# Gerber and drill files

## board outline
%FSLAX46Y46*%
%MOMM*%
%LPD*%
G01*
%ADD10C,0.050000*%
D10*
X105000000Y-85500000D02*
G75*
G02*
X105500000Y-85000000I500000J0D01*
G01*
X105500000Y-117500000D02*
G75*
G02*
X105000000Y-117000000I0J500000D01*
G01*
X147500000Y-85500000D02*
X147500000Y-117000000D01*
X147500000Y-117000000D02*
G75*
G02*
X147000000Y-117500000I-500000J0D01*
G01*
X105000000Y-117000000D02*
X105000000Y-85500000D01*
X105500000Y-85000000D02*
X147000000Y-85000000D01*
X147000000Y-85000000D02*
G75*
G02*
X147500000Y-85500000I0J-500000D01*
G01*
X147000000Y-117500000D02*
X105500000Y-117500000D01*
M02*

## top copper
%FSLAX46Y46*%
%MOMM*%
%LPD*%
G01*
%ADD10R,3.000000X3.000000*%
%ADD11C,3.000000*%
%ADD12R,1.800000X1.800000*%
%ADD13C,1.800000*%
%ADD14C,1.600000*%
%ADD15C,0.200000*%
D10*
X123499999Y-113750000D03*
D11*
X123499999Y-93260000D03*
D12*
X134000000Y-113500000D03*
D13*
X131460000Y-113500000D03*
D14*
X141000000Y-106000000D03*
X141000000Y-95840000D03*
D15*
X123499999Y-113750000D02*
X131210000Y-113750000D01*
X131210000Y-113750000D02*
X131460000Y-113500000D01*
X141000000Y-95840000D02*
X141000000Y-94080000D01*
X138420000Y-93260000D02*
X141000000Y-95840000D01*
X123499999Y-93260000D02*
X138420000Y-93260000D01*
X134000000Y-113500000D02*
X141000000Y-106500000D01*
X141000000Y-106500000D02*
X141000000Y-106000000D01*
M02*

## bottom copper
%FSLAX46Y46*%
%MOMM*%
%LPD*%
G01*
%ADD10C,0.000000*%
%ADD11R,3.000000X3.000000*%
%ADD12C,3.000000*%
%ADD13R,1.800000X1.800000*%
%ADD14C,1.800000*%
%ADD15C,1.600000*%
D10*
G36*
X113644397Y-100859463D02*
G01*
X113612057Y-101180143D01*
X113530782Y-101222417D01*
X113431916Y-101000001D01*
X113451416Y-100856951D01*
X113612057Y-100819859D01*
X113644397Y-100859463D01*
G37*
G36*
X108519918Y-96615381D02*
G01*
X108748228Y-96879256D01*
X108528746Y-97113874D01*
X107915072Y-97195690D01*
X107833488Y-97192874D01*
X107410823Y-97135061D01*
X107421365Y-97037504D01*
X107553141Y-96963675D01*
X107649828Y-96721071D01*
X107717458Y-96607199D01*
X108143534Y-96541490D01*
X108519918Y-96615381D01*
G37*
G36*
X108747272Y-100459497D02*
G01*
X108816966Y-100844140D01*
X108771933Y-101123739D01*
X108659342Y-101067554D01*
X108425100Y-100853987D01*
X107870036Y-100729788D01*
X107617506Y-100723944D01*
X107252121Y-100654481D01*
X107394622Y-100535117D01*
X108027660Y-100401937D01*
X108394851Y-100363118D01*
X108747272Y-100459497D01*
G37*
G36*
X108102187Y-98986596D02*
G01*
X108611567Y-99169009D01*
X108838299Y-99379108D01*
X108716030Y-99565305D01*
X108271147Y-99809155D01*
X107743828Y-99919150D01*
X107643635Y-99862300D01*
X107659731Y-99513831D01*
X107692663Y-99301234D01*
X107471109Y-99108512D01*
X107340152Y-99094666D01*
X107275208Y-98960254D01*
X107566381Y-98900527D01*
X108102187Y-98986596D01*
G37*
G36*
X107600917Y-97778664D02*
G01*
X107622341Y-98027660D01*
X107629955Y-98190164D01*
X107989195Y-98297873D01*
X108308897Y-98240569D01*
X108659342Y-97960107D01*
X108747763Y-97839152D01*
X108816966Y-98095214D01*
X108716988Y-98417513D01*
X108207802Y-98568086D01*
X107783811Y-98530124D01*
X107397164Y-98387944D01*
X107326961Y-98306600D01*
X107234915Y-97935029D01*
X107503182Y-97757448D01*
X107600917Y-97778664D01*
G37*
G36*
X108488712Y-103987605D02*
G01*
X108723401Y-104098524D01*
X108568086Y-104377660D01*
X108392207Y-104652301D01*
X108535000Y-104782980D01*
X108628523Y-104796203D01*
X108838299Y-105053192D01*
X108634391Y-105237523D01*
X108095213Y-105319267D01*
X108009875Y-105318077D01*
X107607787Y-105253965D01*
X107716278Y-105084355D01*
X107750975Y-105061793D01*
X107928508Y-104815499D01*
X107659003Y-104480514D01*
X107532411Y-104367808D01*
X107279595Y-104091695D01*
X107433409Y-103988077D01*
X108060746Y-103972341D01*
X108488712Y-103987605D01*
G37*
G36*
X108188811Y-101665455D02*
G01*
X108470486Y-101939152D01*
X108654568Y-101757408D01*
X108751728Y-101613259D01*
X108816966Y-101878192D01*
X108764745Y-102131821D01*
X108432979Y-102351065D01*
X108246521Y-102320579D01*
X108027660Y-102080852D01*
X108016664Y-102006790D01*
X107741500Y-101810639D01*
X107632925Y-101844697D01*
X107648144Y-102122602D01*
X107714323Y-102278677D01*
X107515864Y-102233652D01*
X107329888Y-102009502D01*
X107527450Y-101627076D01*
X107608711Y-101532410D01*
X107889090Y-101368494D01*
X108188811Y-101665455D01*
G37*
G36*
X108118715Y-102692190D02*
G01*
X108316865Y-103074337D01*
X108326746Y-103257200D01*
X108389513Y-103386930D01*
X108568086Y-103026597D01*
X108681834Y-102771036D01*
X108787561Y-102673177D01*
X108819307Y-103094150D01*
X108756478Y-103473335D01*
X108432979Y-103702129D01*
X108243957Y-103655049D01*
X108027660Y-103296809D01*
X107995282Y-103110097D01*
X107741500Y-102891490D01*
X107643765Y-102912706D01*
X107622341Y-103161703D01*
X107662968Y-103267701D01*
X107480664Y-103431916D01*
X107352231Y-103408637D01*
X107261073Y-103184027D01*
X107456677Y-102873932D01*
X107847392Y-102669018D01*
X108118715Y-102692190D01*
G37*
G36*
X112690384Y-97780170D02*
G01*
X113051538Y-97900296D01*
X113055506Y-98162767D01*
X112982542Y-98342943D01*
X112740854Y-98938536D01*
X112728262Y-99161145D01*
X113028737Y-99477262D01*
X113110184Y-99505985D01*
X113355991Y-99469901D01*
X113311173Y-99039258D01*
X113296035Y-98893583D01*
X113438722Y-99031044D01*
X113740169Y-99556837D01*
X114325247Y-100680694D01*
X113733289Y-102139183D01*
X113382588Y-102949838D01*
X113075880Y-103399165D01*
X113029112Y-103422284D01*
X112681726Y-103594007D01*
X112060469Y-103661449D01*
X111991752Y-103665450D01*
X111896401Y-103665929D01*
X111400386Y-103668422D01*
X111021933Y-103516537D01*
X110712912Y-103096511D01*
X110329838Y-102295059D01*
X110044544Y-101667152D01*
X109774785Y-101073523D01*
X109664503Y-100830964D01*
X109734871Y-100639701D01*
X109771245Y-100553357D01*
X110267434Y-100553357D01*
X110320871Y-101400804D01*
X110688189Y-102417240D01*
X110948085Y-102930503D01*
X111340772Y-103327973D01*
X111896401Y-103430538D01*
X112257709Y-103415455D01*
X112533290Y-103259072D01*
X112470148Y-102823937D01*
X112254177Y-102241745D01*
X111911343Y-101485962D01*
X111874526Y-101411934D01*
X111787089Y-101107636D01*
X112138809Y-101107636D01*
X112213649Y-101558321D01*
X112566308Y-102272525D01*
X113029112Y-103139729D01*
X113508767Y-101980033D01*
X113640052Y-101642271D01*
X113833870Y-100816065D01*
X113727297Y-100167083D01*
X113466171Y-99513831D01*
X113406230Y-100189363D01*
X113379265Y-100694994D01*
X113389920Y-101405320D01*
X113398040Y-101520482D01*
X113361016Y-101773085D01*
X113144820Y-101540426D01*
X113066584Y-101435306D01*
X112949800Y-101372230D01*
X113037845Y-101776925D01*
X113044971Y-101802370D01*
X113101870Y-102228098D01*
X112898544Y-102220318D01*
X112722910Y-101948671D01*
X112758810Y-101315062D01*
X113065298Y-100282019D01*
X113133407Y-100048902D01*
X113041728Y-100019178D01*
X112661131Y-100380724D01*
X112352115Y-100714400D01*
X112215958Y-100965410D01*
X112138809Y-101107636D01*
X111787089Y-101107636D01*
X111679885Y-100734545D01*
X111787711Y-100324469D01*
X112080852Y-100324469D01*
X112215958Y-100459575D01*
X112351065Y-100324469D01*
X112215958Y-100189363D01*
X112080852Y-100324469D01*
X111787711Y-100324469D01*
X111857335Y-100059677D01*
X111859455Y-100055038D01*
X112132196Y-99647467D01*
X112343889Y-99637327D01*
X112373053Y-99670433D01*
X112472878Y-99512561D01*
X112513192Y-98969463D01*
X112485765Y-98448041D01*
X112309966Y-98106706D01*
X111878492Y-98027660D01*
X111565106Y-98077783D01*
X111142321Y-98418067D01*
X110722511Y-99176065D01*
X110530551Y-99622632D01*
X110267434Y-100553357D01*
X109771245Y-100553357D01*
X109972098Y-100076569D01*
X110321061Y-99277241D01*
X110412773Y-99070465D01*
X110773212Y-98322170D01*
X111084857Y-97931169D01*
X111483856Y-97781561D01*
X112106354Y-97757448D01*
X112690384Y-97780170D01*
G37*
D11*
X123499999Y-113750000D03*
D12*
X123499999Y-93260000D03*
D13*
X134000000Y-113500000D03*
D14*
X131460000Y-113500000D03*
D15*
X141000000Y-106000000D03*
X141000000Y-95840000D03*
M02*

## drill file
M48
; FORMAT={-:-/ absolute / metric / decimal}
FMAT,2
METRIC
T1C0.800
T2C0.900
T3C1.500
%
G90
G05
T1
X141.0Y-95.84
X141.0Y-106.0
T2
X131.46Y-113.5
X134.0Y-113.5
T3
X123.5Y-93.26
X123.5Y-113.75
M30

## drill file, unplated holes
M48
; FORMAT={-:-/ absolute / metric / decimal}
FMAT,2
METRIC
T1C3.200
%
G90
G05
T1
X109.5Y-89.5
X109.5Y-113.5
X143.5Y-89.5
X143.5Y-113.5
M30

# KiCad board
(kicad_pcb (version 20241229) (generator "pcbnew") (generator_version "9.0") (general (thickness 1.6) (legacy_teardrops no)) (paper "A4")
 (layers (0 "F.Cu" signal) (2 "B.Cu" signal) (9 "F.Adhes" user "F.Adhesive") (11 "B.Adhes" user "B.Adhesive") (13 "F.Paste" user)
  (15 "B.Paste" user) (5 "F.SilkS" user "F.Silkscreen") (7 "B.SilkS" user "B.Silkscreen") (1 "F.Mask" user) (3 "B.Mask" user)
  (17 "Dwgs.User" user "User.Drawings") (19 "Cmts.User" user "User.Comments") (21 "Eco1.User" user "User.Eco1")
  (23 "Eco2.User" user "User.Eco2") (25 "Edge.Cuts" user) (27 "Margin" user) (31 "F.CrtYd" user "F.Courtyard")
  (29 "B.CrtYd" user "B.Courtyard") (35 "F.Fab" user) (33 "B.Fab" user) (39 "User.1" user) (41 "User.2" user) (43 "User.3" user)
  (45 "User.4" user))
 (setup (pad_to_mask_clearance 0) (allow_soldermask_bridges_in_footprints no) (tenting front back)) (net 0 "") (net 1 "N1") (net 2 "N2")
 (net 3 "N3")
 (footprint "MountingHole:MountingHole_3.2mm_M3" (layer "F.Cu") (at 143.5 89.5)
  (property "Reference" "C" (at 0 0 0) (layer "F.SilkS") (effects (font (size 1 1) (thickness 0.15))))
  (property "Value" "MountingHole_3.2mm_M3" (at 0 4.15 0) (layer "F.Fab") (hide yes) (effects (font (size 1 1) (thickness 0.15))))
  (pad "" np_thru_hole circle (at 0 0) (size 3.2 3.2) (drill 3.2) (layers "*.Cu" "*.Mask")))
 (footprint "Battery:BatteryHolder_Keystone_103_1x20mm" (layer "F.Cu") (at 123.499999 113.75 90)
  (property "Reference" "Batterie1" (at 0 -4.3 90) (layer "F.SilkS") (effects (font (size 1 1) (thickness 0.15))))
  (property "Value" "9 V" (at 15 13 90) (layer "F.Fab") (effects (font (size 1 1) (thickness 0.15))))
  (pad "1" thru_hole rect (at 0 0 90) (size 3 3) (drill 1.5) (layers "*.Cu" "*.Mask") (remove_unused_layers no) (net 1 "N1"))
  (pad "2" thru_hole circle (at 20.49 0 90) (size 3 3) (drill 1.5) (layers "*.Cu" "*.Mask") (remove_unused_layers no) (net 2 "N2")))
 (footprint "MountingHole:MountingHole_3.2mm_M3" (layer "F.Cu") (at 143.5 113.5)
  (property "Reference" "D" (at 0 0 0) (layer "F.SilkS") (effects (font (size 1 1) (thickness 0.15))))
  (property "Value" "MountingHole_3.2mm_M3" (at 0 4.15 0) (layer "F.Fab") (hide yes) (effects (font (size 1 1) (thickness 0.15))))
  (pad "" np_thru_hole circle (at 0 0) (size 3.2 3.2) (drill 3.2) (layers "*.Cu" "*.Mask")))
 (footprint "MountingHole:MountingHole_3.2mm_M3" (layer "F.Cu") (at 109.5 113.5)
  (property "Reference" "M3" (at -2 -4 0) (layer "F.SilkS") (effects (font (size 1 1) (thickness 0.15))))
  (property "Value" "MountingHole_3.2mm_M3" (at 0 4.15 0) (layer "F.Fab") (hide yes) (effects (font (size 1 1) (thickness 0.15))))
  (pad "" np_thru_hole circle (at 0 0) (size 3.2 3.2) (drill 3.2) (layers "*.Cu" "*.Mask")))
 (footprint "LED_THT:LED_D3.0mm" (layer "F.Cu") (at 134 113.5 180)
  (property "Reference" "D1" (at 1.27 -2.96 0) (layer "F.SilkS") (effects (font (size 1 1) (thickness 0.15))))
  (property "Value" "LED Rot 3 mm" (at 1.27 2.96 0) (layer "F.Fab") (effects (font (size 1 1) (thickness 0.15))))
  (pad "1" thru_hole rect (at 0 0 180) (size 1.8 1.8) (drill 0.9) (layers "*.Cu" "*.Mask") (remove_unused_layers no) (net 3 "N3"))
  (pad "2" thru_hole circle (at 2.54 0 180) (size 1.8 1.8) (drill 0.9) (layers "*.Cu" "*.Mask") (remove_unused_layers no) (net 1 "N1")))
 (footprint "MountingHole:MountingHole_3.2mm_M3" (layer "F.Cu") (at 109.5 89.5)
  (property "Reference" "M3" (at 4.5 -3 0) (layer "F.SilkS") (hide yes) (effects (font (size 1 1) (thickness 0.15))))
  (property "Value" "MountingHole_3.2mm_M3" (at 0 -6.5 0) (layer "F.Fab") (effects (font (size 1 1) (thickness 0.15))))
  (pad "" np_thru_hole circle (at 0 0) (size 3.2 3.2) (drill 3.2) (layers "*.Cu" "*.Mask")))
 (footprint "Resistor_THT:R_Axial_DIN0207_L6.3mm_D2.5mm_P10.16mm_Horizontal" (layer "F.Cu") (at 141 106 90)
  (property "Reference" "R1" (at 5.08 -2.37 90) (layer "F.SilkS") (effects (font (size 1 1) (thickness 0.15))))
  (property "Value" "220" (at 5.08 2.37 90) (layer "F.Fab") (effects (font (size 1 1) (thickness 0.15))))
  (pad "1" thru_hole circle (at 0 0 90) (size 1.6 1.6) (drill 0.8) (layers "*.Cu" "*.Mask") (remove_unused_layers no) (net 3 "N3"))
  (pad "2" thru_hole circle (at 10.16 0 90) (size 1.6 1.6) (drill 0.8) (layers "*.Cu" "*.Mask") (remove_unused_layers no) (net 2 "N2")))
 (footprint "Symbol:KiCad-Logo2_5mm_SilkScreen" (layer "B.Cu") (at 124 99 180)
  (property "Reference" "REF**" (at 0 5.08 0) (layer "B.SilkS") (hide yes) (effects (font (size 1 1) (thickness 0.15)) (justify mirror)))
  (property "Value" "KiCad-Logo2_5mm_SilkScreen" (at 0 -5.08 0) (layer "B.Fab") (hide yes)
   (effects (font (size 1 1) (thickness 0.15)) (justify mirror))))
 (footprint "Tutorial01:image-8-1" (layer "B.Cu") (at 111 101 90)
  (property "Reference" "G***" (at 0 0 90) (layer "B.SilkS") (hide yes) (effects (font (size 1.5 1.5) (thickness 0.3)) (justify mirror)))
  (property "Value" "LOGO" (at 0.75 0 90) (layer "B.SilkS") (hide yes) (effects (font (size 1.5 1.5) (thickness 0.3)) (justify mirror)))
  (fp_poly
   (pts (xy 0.180141 2.612057) (xy 0.143049 2.451416) (xy -0.000001 2.431916) (xy -0.222417 2.530782) (xy -0.180143 2.612057)
    (xy 0.140537 2.644397))
   (stroke (width 0) (type solid)) (fill yes) (layer "B.Cu"))
  (fp_poly
   (pts (xy 4.384619 -2.480082) (xy 4.45851 -2.856466) (xy 4.392801 -3.282542) (xy 4.278929 -3.350172) (xy 4.036325 -3.446859)
    (xy 3.962496 -3.578635) (xy 3.864939 -3.589177) (xy 3.807126 -3.166512) (xy 3.80431 -3.084928) (xy 3.886126 -2.471254)
    (xy 4.120744 -2.251772))
   (stroke (width 0) (type solid)) (fill yes) (layer "B.Cu"))
  (fp_poly
   (pts (xy 0.540503 -2.252728) (xy 0.636882 -2.605149) (xy 0.598063 -2.97234) (xy 0.464883 -3.605378) (xy 0.345519 -3.747879)
    (xy 0.276056 -3.382494) (xy 0.270212 -3.129964) (xy 0.146013 -2.5749) (xy -0.067554 -2.340658) (xy -0.123739 -2.228067)
    (xy 0.15586 -2.183034))
   (stroke (width 0) (type solid)) (fill yes) (layer "B.Cu"))
  (fp_poly
   (pts (xy 1.830991 -2.388433) (xy 2.013404 -2.897813) (xy 2.099473 -3.433619) (xy 2.039746 -3.724792) (xy 1.905334 -3.659848)
    (xy 1.891488 -3.528891) (xy 1.698766 -3.307337) (xy 1.486169 -3.340269) (xy 1.1377 -3.356365) (xy 1.08085 -3.256172)
    (xy 1.190845 -2.728853) (xy 1.434695 -2.28397) (xy 1.620892 -2.161701))
   (stroke (width 0) (type solid)) (fill yes) (layer "B.Cu"))
  (fp_poly
   (pts (xy 3.160848 -2.252237) (xy 3.039893 -2.340658) (xy 2.759431 -2.691103) (xy 2.702127 -3.010805) (xy 2.809836 -3.370045)
    (xy 2.97234 -3.377659) (xy 3.221336 -3.399083) (xy 3.242552 -3.496818) (xy 3.064971 -3.765085) (xy 2.6934 -3.673039)
    (xy 2.612056 -3.602836) (xy 2.469876 -3.216189) (xy 2.431914 -2.792198) (xy 2.582487 -2.283012) (xy 2.904786 -2.183034))
   (stroke (width 0) (type solid)) (fill yes) (layer "B.Cu"))
  (fp_poly
   (pts (xy -3.796203 -2.371477) (xy -3.78298 -2.465) (xy -3.652301 -2.607793) (xy -3.37766 -2.431914) (xy -3.098524 -2.276599)
    (xy -2.987605 -2.511288) (xy -2.972341 -2.939254) (xy -2.988077 -3.566591) (xy -3.091695 -3.720405) (xy -3.367808 -3.467589)
    (xy -3.480514 -3.340997) (xy -3.815499 -3.071492) (xy -4.061793 -3.249025) (xy -4.084355 -3.283722) (xy -4.253965 -3.392213)
    (xy -4.318077 -2.990125) (xy -4.319267 -2.904787) (xy -4.237523 -2.365609) (xy -4.053192 -2.161701))
   (stroke (width 0) (type solid)) (fill yes) (layer "B.Cu"))
  (fp_poly
   (pts (xy -0.613259 -2.248272) (xy -0.757408 -2.345432) (xy -0.939152 -2.529514) (xy -0.665455 -2.811189) (xy -0.368494 -3.11091)
    (xy -0.53241 -3.391289) (xy -0.627076 -3.47255) (xy -1.009502 -3.670112) (xy -1.233652 -3.484136) (xy -1.278677 -3.285677)
    (xy -1.122602 -3.351856) (xy -0.844697 -3.367075) (xy -0.810639 -3.2585) (xy -1.00679 -2.983336) (xy -1.080852 -2.97234)
    (xy -1.320579 -2.753479) (xy -1.351065 -2.567021) (xy -1.131821 -2.235255) (xy -0.878192 -2.183034))
   (stroke (width 0) (type solid)) (fill yes) (layer "B.Cu"))
  (fp_poly
   (pts (xy -1.673177 -2.212439) (xy -1.771036 -2.318166) (xy -2.026597 -2.431914) (xy -2.38693 -2.610487) (xy -2.2572 -2.673254)
    (xy -2.074337 -2.683135) (xy -1.69219 -2.881285) (xy -1.669018 -3.152608) (xy -1.873932 -3.543323) (xy -2.184027 -3.738927)
    (xy -2.408637 -3.647769) (xy -2.431916 -3.519336) (xy -2.267701 -3.337032) (xy -2.161703 -3.377659) (xy -1.912706 -3.356235)
    (xy -1.89149 -3.2585) (xy -2.110097 -3.004718) (xy -2.296809 -2.97234) (xy -2.655049 -2.756043) (xy -2.702129 -2.567021)
    (xy -2.473335 -2.243522) (xy -2.09415 -2.180693))
   (stroke (width 0) (type solid)) (fill yes) (layer "B.Cu"))
  (fp_poly
   (pts (xy 1.443163 2.740169) (xy 1.968956 2.438722) (xy 2.106417 2.296035) (xy 1.960742 2.311173) (xy 1.530099 2.355991)
    (xy 1.494015 2.110184) (xy 1.522738 2.028737) (xy 1.838855 1.728262) (xy 2.061464 1.740854) (xy 2.657057 1.982542)
    (xy 2.837233 2.055506) (xy 3.099704 2.051538) (xy 3.21983 1.690384) (xy 3.242552 1.106354) (xy 3.218439 0.483856) (xy 3.068831 0.084857)
    (xy 2.67783 -0.226788) (xy 1.929535 -0.587227) (xy 1.722759 -0.678939) (xy 0.923431 -1.027902) (xy 0.360299 -1.265129)
    (xy 0.169036 -1.335497) (xy -0.073523 -1.225215) (xy -0.667152 -0.955456) (xy -1.295059 -0.670162) (xy -2.096511 -0.287088)
    (xy -2.516537 0.021933) (xy -2.668422 0.400386) (xy -2.665929 0.896401) (xy -2.430538 0.896401) (xy -2.327973 0.340772)
    (xy -1.930503 -0.051915) (xy -1.41724 -0.311811) (xy -0.400804 -0.679129) (xy 0.446643 -0.732566) (xy 1.377368 -0.469449)
    (xy 1.823935 -0.277489) (xy 2.581933 0.142321) (xy 2.922217 0.565106) (xy 2.97234 0.878492) (xy 2.893294 1.309966)
    (xy 2.551959 1.485765) (xy 2.030537 1.513192) (xy 1.487439 1.472878) (xy 1.329567 1.373053) (xy 1.362673 1.343889)
    (xy 1.352533 1.132196) (xy 0.944962 0.859455) (xy 0.940323 0.857335) (xy 0.265455 0.679885) (xy -0.411934 0.874526)
    (xy -0.485962 0.911343) (xy -1.241745 1.254177) (xy -1.823937 1.470148) (xy -2.259072 1.53329) (xy -2.415455 1.257709)
    (xy -2.430538 0.896401) (xy -2.665929 0.896401) (xy -2.66545 0.991752) (xy -2.661449 1.060469) (xy -2.594007 1.681726)
    (xy -2.422284 2.029112) (xy -2.139729 2.029112) (xy -1.272525 1.566308) (xy -0.558321 1.213649) (xy -0.107636 1.138809)
    (xy 0.03459 1.215958) (xy 0.540425 1.215958) (xy 0.675531 1.080852) (xy 0.810637 1.215958) (xy 0.675531 1.351065) (xy 0.540425 1.215958)
    (xy 0.03459 1.215958) (xy 0.2856 1.352115) (xy 0.619276 1.661131) (xy 0.980822 2.041728) (xy 0.951098 2.133407) (xy 0.717981 2.065298)
    (xy -0.315062 1.75881) (xy -0.948671 1.72291) (xy -1.220318 1.898544) (xy -1.228098 2.10187) (xy -0.80237 2.044971)
    (xy -0.776925 2.037845) (xy -0.37223 1.9498) (xy -0.435306 2.066584) (xy -0.540426 2.14482) (xy -0.773085 2.361016)
    (xy -0.520482 2.39804) (xy -0.40532 2.38992) (xy 0.305006 2.379265) (xy 0.810637 2.40623) (xy 1.486169 2.466171) (xy 0.832917 2.727297)
    (xy 0.183935 2.83387) (xy -0.642271 2.640052) (xy -0.980033 2.508767) (xy -2.139729 2.029112) (xy -2.422284 2.029112)
    (xy -2.399165 2.07588) (xy -1.949838 2.382588) (xy -1.139183 2.733289) (xy 0.319306 3.325247))
   (stroke (width 0) (type solid)) (fill yes) (layer "B.Cu")))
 (gr_arc (start 105 85.5) (mid 105.146447 85.146447) (end 105.5 85) (stroke (width 0.05) (type default)) (layer "Edge.Cuts"))
 (gr_arc (start 105.5 117.5) (mid 105.146447 117.353553) (end 105 117) (stroke (width 0.05) (type default)) (layer "Edge.Cuts"))
 (gr_line (start 147.5 85.5) (end 147.5 117) (stroke (width 0.05) (type default)) (layer "Edge.Cuts"))
 (gr_arc (start 147.5 117) (mid 147.353553 117.353553) (end 147 117.5) (stroke (width 0.05) (type default)) (layer "Edge.Cuts"))
 (gr_line (start 105 117) (end 105 85.5) (stroke (width 0.05) (type default)) (layer "Edge.Cuts"))
 (gr_line (start 105.5 85) (end 147 85) (stroke (width 0.05) (type default)) (layer "Edge.Cuts"))
 (gr_arc (start 147 85) (mid 147.353553 85.146447) (end 147.5 85.5) (stroke (width 0.05) (type default)) (layer "Edge.Cuts"))
 (gr_line (start 147 117.5) (end 105.5 117.5) (stroke (width 0.05) (type default)) (layer "Edge.Cuts"))
 (segment (start 123.499999 113.75) (end 131.21 113.75) (width 0.2) (layer "F.Cu") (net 1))
 (segment (start 131.21 113.75) (end 131.46 113.5) (width 0.2) (layer "F.Cu") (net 1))
 (segment (start 141 95.84) (end 141 94.08) (width 0.2) (layer "F.Cu") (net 2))
 (segment (start 138.42 93.26) (end 141 95.84) (width 0.2) (layer "F.Cu") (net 2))
 (segment (start 123.499999 93.26) (end 138.42 93.26) (width 0.2) (layer "F.Cu") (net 2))
 (segment (start 134 113.5) (end 141 106.5) (width 0.2) (layer "F.Cu") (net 3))
 (segment (start 141 106.5) (end 141 106) (width 0.2) (layer "F.Cu") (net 3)))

